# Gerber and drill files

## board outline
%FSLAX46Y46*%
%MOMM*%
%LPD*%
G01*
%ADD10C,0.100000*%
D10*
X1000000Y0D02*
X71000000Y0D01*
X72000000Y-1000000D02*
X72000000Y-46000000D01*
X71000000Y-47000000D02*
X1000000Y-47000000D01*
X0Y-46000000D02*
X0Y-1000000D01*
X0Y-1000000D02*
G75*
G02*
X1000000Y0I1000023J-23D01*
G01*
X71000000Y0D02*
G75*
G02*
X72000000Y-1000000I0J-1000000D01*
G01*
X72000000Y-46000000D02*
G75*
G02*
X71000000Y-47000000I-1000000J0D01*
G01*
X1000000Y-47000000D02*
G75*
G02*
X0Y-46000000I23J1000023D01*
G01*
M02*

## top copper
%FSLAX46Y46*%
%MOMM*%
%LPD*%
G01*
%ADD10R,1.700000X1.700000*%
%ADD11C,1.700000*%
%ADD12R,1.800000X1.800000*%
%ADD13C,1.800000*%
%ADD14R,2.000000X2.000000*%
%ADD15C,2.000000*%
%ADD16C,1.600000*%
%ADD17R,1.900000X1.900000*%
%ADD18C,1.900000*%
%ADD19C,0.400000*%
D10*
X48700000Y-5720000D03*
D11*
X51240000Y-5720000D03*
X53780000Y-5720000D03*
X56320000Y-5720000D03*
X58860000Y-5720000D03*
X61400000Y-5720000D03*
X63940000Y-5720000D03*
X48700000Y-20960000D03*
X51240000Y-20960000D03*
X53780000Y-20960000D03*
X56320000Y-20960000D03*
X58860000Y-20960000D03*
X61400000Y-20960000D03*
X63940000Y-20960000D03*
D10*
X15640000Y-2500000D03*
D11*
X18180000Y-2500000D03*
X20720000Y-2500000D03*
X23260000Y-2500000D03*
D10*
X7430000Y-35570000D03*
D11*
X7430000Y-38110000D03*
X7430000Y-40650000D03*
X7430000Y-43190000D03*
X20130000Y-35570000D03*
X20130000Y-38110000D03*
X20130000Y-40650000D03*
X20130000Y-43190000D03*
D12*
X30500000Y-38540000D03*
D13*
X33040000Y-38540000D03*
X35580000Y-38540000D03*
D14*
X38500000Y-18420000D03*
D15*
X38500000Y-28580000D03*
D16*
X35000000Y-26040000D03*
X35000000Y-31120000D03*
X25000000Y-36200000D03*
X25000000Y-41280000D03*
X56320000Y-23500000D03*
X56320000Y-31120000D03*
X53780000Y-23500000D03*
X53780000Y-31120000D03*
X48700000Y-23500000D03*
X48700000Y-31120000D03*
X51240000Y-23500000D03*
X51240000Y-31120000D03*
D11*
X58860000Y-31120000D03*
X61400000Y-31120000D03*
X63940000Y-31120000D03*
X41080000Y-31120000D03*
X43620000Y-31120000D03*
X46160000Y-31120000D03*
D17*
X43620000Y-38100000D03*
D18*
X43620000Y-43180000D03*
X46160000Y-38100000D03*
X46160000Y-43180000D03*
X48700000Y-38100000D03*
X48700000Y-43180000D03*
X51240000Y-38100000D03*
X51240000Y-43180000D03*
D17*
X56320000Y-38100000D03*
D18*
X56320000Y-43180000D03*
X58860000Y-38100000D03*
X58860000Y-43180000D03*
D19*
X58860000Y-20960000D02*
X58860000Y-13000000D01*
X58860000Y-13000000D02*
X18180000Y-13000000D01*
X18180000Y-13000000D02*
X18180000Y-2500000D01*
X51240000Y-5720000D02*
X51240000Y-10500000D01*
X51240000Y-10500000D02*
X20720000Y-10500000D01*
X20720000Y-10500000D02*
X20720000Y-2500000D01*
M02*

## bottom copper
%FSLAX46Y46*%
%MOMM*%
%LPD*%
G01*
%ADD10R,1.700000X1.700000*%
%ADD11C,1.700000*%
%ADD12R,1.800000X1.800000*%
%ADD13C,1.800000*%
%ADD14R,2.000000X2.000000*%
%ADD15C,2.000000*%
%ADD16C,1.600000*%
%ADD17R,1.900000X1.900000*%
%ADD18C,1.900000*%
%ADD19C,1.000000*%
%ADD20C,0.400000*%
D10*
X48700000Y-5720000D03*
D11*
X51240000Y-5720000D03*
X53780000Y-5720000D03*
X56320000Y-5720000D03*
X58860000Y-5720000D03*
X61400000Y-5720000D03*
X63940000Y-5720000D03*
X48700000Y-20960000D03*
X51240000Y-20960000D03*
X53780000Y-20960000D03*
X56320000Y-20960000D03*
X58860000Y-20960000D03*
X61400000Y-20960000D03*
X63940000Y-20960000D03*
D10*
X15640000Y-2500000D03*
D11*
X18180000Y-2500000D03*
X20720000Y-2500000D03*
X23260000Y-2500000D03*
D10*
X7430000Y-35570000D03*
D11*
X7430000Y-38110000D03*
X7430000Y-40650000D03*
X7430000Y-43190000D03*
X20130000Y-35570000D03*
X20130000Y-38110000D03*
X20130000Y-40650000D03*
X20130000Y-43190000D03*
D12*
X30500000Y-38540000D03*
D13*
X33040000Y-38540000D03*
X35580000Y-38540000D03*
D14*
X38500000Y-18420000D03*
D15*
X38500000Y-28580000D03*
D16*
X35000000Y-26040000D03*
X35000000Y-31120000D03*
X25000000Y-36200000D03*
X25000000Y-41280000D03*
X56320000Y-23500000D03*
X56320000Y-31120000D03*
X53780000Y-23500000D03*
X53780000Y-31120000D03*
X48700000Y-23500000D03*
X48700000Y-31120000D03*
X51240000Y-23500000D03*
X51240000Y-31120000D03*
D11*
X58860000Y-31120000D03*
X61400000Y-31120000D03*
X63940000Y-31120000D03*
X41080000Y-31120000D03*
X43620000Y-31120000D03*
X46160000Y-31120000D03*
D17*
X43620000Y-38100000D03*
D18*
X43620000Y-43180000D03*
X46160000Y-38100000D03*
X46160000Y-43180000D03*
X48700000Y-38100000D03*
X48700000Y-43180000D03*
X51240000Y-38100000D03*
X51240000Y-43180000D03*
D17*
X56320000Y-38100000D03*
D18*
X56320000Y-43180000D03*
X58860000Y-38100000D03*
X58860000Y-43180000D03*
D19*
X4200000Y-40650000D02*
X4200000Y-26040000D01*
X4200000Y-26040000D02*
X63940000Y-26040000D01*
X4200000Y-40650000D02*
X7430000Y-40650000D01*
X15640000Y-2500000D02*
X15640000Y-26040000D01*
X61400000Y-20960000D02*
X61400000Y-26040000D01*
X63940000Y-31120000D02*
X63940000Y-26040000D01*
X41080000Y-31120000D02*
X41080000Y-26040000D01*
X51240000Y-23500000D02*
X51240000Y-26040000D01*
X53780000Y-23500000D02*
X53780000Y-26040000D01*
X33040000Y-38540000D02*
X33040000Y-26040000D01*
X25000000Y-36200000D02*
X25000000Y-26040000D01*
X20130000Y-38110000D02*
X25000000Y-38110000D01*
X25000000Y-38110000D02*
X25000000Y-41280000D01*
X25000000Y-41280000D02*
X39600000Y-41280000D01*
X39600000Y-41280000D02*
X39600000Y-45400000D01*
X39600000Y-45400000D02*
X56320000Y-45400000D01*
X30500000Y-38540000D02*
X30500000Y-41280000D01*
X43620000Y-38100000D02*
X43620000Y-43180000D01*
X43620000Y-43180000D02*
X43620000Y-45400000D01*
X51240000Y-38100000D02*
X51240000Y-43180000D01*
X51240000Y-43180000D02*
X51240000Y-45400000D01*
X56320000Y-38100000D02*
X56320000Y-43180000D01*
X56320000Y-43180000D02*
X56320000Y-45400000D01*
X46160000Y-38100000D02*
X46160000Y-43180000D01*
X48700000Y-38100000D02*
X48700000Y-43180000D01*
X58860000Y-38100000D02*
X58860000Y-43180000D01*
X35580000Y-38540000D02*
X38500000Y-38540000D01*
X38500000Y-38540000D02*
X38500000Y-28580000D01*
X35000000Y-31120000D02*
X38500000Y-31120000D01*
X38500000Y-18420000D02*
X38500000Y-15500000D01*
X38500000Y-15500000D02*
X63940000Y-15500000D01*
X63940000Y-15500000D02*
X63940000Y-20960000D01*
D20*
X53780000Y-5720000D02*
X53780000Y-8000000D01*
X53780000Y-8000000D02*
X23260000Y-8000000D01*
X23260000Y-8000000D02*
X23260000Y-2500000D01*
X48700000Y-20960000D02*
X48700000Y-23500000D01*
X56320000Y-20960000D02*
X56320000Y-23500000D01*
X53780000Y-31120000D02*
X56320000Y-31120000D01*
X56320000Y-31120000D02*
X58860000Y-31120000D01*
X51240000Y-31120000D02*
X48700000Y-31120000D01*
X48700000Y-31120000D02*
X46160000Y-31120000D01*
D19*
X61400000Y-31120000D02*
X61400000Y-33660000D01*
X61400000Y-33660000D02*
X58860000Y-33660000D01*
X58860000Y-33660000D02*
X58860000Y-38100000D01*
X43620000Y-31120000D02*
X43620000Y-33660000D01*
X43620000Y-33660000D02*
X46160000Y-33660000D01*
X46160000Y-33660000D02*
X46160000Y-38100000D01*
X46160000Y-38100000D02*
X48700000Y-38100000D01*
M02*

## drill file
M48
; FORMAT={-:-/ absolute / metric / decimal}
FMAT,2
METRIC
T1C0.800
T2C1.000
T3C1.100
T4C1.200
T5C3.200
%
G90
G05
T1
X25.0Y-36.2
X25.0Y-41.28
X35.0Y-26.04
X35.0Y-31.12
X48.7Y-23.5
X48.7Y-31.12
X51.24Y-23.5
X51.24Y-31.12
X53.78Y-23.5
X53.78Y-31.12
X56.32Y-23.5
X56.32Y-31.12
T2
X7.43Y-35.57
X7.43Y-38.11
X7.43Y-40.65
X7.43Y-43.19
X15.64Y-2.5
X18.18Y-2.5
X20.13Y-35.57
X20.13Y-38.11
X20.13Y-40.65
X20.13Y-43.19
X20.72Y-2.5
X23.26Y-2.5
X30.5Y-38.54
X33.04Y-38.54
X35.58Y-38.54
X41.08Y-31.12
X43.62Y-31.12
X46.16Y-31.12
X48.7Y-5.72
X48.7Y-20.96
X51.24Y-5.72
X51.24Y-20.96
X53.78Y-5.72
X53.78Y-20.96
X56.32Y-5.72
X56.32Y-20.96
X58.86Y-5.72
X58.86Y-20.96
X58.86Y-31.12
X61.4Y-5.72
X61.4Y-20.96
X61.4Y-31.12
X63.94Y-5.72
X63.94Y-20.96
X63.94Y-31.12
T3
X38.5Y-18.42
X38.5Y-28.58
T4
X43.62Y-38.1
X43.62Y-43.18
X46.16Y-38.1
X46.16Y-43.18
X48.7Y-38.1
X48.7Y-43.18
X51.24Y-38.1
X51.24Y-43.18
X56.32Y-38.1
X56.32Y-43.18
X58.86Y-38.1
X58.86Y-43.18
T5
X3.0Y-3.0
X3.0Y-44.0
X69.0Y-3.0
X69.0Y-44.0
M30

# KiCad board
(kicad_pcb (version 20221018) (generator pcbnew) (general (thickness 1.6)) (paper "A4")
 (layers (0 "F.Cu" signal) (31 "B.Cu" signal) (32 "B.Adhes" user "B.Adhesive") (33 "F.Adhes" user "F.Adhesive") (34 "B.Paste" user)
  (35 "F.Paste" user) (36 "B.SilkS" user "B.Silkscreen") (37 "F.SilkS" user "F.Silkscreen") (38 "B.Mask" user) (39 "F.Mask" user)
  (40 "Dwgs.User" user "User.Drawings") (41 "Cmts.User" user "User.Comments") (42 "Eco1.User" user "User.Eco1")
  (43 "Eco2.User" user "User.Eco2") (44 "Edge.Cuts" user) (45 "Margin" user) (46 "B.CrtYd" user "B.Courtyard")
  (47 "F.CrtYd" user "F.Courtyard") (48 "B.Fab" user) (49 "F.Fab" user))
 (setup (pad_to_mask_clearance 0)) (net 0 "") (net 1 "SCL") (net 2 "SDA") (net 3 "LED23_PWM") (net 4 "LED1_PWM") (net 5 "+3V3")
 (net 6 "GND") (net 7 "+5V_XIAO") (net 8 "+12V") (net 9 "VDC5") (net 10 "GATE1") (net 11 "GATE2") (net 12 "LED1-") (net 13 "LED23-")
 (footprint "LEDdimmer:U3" (layer "F.Cu") (at 0 0)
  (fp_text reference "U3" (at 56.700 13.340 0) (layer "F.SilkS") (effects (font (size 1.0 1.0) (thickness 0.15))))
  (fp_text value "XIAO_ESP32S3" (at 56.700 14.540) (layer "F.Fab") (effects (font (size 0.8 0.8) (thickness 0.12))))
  (pad "1" thru_hole rect (at 48.7 5.72) (size 1.7 1.7) (drill 1.0) (layers "*.Cu" "*.Mask"))
  (pad "2" thru_hole circle (at 51.24 5.72) (size 1.7 1.7) (drill 1.0) (layers "*.Cu" "*.Mask") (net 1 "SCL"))
  (pad "3" thru_hole circle (at 53.78 5.72) (size 1.7 1.7) (drill 1.0) (layers "*.Cu" "*.Mask") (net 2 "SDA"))
  (pad "4" thru_hole circle (at 56.32 5.72) (size 1.7 1.7) (drill 1.0) (layers "*.Cu" "*.Mask"))
  (pad "5" thru_hole circle (at 58.86 5.72) (size 1.7 1.7) (drill 1.0) (layers "*.Cu" "*.Mask"))
  (pad "6" thru_hole circle (at 61.4 5.72) (size 1.7 1.7) (drill 1.0) (layers "*.Cu" "*.Mask"))
  (pad "7" thru_hole circle (at 63.94 5.72) (size 1.7 1.7) (drill 1.0) (layers "*.Cu" "*.Mask"))
  (pad "8" thru_hole circle (at 48.7 20.96) (size 1.7 1.7) (drill 1.0) (layers "*.Cu" "*.Mask") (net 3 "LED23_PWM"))
  (pad "9" thru_hole circle (at 51.24 20.96) (size 1.7 1.7) (drill 1.0) (layers "*.Cu" "*.Mask"))
  (pad "10" thru_hole circle (at 53.78 20.96) (size 1.7 1.7) (drill 1.0) (layers "*.Cu" "*.Mask"))
  (pad "11" thru_hole circle (at 56.32 20.96) (size 1.7 1.7) (drill 1.0) (layers "*.Cu" "*.Mask") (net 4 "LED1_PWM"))
  (pad "12" thru_hole circle (at 58.86 20.96) (size 1.7 1.7) (drill 1.0) (layers "*.Cu" "*.Mask") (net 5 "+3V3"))
  (pad "13" thru_hole circle (at 61.4 20.96) (size 1.7 1.7) (drill 1.0) (layers "*.Cu" "*.Mask") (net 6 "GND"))
  (pad "14" thru_hole circle (at 63.94 20.96) (size 1.7 1.7) (drill 1.0) (layers "*.Cu" "*.Mask") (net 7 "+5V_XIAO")))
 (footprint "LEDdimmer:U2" (layer "F.Cu") (at 0 0)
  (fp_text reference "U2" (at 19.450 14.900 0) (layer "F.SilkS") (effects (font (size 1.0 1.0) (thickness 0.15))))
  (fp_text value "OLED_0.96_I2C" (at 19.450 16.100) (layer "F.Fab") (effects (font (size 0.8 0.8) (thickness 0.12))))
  (pad "1" thru_hole rect (at 15.64 2.5) (size 1.7 1.7) (drill 1.0) (layers "*.Cu" "*.Mask") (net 6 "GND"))
  (pad "2" thru_hole circle (at 18.18 2.5) (size 1.7 1.7) (drill 1.0) (layers "*.Cu" "*.Mask") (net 5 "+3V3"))
  (pad "3" thru_hole circle (at 20.72 2.5) (size 1.7 1.7) (drill 1.0) (layers "*.Cu" "*.Mask") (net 1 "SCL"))
  (pad "4" thru_hole circle (at 23.26 2.5) (size 1.7 1.7) (drill 1.0) (layers "*.Cu" "*.Mask") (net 2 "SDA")))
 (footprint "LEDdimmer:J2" (layer "F.Cu") (at 0 0)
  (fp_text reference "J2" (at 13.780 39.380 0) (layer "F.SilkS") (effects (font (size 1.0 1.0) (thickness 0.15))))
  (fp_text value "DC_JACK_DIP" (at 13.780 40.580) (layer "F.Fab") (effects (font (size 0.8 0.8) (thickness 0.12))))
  (pad "1" thru_hole rect (at 7.43 35.57) (size 1.7 1.7) (drill 1.0) (layers "*.Cu" "*.Mask") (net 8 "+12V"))
  (pad "2" thru_hole circle (at 7.43 38.11) (size 1.7 1.7) (drill 1.0) (layers "*.Cu" "*.Mask") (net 8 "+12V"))
  (pad "3" thru_hole circle (at 7.43 40.65) (size 1.7 1.7) (drill 1.0) (layers "*.Cu" "*.Mask") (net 6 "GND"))
  (pad "4" thru_hole circle (at 7.43 43.19) (size 1.7 1.7) (drill 1.0) (layers "*.Cu" "*.Mask") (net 6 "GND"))
  (pad "5" thru_hole circle (at 20.13 35.57) (size 1.7 1.7) (drill 1.0) (layers "*.Cu" "*.Mask") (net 8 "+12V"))
  (pad "6" thru_hole circle (at 20.13 38.11) (size 1.7 1.7) (drill 1.0) (layers "*.Cu" "*.Mask") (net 8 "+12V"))
  (pad "7" thru_hole circle (at 20.13 40.65) (size 1.7 1.7) (drill 1.0) (layers "*.Cu" "*.Mask") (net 6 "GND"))
  (pad "8" thru_hole circle (at 20.13 43.19) (size 1.7 1.7) (drill 1.0) (layers "*.Cu" "*.Mask") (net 6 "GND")))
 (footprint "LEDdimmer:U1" (layer "F.Cu") (at 0 0)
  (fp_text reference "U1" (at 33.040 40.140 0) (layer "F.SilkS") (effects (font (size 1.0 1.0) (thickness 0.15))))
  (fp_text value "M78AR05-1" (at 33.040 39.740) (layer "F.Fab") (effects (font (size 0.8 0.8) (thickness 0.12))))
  (pad "1" thru_hole rect (at 30.5 38.54) (size 1.8 1.8) (drill 1.0) (layers "*.Cu" "*.Mask") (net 8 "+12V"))
  (pad "2" thru_hole circle (at 33.04 38.54) (size 1.8 1.8) (drill 1.0) (layers "*.Cu" "*.Mask") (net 6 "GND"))
  (pad "3" thru_hole circle (at 35.58 38.54) (size 1.8 1.8) (drill 1.0) (layers "*.Cu" "*.Mask") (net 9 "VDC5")))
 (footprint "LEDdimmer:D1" (layer "F.Cu") (at 0 0)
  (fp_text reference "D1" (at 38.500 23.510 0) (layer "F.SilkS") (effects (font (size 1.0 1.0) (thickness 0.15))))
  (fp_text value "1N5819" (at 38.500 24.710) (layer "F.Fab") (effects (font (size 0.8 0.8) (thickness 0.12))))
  (pad "1" thru_hole rect (at 38.5 18.42) (size 2.0 2.0) (drill 1.1) (layers "*.Cu" "*.Mask") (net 7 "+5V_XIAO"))
  (pad "2" thru_hole circle (at 38.5 28.58) (size 2.0 2.0) (drill 1.1) (layers "*.Cu" "*.Mask") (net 9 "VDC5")))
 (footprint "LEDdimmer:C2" (layer "F.Cu") (at 0 0)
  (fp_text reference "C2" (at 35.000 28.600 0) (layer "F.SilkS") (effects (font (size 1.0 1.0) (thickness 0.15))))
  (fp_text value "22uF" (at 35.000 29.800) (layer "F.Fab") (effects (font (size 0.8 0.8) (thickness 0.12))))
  (pad "1" thru_hole circle (at 35.0 26.04) (size 1.6 1.6) (drill 0.8) (layers "*.Cu" "*.Mask") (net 6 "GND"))
  (pad "2" thru_hole circle (at 35.0 31.12) (size 1.6 1.6) (drill 0.8) (layers "*.Cu" "*.Mask") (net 9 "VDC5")))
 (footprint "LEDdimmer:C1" (layer "F.Cu") (at 0 0)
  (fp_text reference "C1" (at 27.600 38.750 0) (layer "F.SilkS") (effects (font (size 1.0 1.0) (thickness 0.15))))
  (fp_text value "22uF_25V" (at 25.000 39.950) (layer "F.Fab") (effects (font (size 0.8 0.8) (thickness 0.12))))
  (pad "1" thru_hole circle (at 25.0 36.2) (size 1.6 1.6) (drill 0.8) (layers "*.Cu" "*.Mask") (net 6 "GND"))
  (pad "2" thru_hole circle (at 25.0 41.28) (size 1.6 1.6) (drill 0.8) (layers "*.Cu" "*.Mask") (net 8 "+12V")))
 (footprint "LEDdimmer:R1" (layer "F.Cu") (at 0 0)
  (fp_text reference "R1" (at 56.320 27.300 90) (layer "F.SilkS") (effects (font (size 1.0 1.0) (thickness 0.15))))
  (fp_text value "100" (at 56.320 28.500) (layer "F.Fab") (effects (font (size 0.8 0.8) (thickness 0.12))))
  (pad "1" thru_hole circle (at 56.32 23.5) (size 1.6 1.6) (drill 0.8) (layers "*.Cu" "*.Mask") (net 4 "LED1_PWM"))
  (pad "2" thru_hole circle (at 56.32 31.12) (size 1.6 1.6) (drill 0.8) (layers "*.Cu" "*.Mask") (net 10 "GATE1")))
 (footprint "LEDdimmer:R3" (layer "F.Cu") (at 0 0)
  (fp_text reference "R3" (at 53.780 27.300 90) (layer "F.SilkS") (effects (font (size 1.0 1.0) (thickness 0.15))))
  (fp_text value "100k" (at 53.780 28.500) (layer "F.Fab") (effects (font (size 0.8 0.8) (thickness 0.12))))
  (pad "1" thru_hole circle (at 53.78 23.5) (size 1.6 1.6) (drill 0.8) (layers "*.Cu" "*.Mask") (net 6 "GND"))
  (pad "2" thru_hole circle (at 53.78 31.12) (size 1.6 1.6) (drill 0.8) (layers "*.Cu" "*.Mask") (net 10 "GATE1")))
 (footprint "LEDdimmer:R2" (layer "F.Cu") (at 0 0)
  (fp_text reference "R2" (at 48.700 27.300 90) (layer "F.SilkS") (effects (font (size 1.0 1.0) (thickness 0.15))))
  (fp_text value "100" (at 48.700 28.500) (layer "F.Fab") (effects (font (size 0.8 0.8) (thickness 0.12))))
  (pad "1" thru_hole circle (at 48.7 23.5) (size 1.6 1.6) (drill 0.8) (layers "*.Cu" "*.Mask") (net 3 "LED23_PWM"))
  (pad "2" thru_hole circle (at 48.7 31.12) (size 1.6 1.6) (drill 0.8) (layers "*.Cu" "*.Mask") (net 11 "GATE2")))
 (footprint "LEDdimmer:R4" (layer "F.Cu") (at 0 0)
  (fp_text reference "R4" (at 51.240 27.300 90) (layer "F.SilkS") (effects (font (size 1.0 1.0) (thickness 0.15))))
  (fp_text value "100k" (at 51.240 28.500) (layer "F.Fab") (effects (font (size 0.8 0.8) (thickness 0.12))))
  (pad "1" thru_hole circle (at 51.24 23.5) (size 1.6 1.6) (drill 0.8) (layers "*.Cu" "*.Mask") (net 6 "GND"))
  (pad "2" thru_hole circle (at 51.24 31.12) (size 1.6 1.6) (drill 0.8) (layers "*.Cu" "*.Mask") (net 11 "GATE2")))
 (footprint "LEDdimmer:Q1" (layer "F.Cu") (at 0 0)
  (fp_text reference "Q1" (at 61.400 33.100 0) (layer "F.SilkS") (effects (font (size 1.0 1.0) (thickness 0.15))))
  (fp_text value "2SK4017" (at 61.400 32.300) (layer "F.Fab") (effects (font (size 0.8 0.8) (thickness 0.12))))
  (pad "1" thru_hole circle (at 58.86 31.12) (size 1.7 1.7) (drill 1.0) (layers "*.Cu" "*.Mask") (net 10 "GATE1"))
  (pad "2" thru_hole circle (at 61.4 31.12) (size 1.7 1.7) (drill 1.0) (layers "*.Cu" "*.Mask") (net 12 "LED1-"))
  (pad "3" thru_hole circle (at 63.94 31.12) (size 1.7 1.7) (drill 1.0) (layers "*.Cu" "*.Mask") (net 6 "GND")))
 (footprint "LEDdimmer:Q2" (layer "F.Cu") (at 0 0)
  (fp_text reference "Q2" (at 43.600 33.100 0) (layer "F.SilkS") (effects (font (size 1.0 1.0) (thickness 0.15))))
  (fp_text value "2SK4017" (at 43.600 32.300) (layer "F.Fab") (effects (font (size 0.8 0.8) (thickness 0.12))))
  (pad "1" thru_hole circle (at 41.08 31.12) (size 1.7 1.7) (drill 1.0) (layers "*.Cu" "*.Mask") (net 6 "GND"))
  (pad "2" thru_hole circle (at 43.62 31.12) (size 1.7 1.7) (drill 1.0) (layers "*.Cu" "*.Mask") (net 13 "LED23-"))
  (pad "3" thru_hole circle (at 46.16 31.12) (size 1.7 1.7) (drill 1.0) (layers "*.Cu" "*.Mask") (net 11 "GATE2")))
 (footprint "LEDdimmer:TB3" (layer "F.Cu") (at 0 0)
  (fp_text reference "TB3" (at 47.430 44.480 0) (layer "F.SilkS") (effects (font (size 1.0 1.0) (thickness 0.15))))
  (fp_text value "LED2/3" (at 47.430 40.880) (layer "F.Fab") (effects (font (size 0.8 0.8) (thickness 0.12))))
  (pad "1" thru_hole rect (at 43.62 38.1) (size 1.9 1.9) (drill 1.2) (layers "*.Cu" "*.Mask") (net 8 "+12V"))
  (pad "2" thru_hole circle (at 43.62 43.18) (size 1.9 1.9) (drill 1.2) (layers "*.Cu" "*.Mask") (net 8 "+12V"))
  (pad "3" thru_hole circle (at 46.16 38.1) (size 1.9 1.9) (drill 1.2) (layers "*.Cu" "*.Mask") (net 13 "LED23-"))
  (pad "4" thru_hole circle (at 46.16 43.18) (size 1.9 1.9) (drill 1.2) (layers "*.Cu" "*.Mask") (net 13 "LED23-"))
  (pad "5" thru_hole circle (at 48.7 38.1) (size 1.9 1.9) (drill 1.2) (layers "*.Cu" "*.Mask") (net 13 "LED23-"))
  (pad "6" thru_hole circle (at 48.7 43.18) (size 1.9 1.9) (drill 1.2) (layers "*.Cu" "*.Mask") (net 13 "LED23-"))
  (pad "7" thru_hole circle (at 51.24 38.1) (size 1.9 1.9) (drill 1.2) (layers "*.Cu" "*.Mask") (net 8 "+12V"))
  (pad "8" thru_hole circle (at 51.24 43.18) (size 1.9 1.9) (drill 1.2) (layers "*.Cu" "*.Mask") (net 8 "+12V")))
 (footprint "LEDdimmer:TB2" (layer "F.Cu") (at 0 0)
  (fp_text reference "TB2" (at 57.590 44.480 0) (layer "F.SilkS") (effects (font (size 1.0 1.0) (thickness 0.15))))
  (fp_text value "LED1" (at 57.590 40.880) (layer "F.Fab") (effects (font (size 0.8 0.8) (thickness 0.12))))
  (pad "1" thru_hole rect (at 56.32 38.1) (size 1.9 1.9) (drill 1.2) (layers "*.Cu" "*.Mask") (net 8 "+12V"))
  (pad "2" thru_hole circle (at 56.32 43.18) (size 1.9 1.9) (drill 1.2) (layers "*.Cu" "*.Mask") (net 8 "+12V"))
  (pad "3" thru_hole circle (at 58.86 38.1) (size 1.9 1.9) (drill 1.2) (layers "*.Cu" "*.Mask") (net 12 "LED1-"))
  (pad "4" thru_hole circle (at 58.86 43.18) (size 1.9 1.9) (drill 1.2) (layers "*.Cu" "*.Mask") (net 12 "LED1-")))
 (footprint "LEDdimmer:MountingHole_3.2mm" (layer "F.Cu") (at 3.0 3.0)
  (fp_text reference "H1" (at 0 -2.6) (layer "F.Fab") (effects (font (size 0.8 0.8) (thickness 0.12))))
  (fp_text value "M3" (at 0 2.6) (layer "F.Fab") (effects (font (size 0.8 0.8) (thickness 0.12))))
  (pad "" np_thru_hole circle (at 0 0) (size 3.2 3.2) (drill 3.2) (layers "*.Cu" "*.Mask")))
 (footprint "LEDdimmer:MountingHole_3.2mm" (layer "F.Cu") (at 69.0 3.0)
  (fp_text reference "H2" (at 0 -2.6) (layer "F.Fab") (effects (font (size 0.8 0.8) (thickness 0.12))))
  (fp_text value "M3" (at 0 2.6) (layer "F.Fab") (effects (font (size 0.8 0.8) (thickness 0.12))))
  (pad "" np_thru_hole circle (at 0 0) (size 3.2 3.2) (drill 3.2) (layers "*.Cu" "*.Mask")))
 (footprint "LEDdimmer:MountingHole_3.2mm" (layer "F.Cu") (at 3.0 44.0)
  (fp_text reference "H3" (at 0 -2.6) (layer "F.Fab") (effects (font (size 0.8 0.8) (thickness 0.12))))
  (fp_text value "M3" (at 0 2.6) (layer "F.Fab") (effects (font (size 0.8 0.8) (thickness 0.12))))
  (pad "" np_thru_hole circle (at 0 0) (size 3.2 3.2) (drill 3.2) (layers "*.Cu" "*.Mask")))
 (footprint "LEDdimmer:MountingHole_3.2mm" (layer "F.Cu") (at 69.0 44.0)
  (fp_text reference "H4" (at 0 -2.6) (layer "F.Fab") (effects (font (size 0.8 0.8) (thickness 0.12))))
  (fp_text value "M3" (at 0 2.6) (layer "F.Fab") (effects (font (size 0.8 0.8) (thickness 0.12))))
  (pad "" np_thru_hole circle (at 0 0) (size 3.2 3.2) (drill 3.2) (layers "*.Cu" "*.Mask")))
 (gr_line (start 1.0 0) (end 71.0 0) (stroke (width 0.1) (type solid)) (layer "Edge.Cuts"))
 (gr_line (start 72.0 1.0) (end 72.0 46.0) (stroke (width 0.1) (type solid)) (layer "Edge.Cuts"))
 (gr_line (start 71.0 47.0) (end 1.0 47.0) (stroke (width 0.1) (type solid)) (layer "Edge.Cuts"))
 (gr_line (start 0 46.0) (end 0 1.0) (stroke (width 0.1) (type solid)) (layer "Edge.Cuts"))
 (gr_arc (start 1.0 0) (mid 0.2929 0.2929) (end 0 1.0) (stroke (width 0.1) (type solid)) (layer "Edge.Cuts"))
 (gr_arc (start 72.0 1.0) (mid 71.7071 0.2929) (end 71.0 0) (stroke (width 0.1) (type solid)) (layer "Edge.Cuts"))
 (gr_arc (start 71.0 47.0) (mid 71.7071 46.7071) (end 72.0 46.0) (stroke (width 0.1) (type solid)) (layer "Edge.Cuts"))
 (gr_arc (start 0 46.0) (mid 0.2929 46.7071) (end 1.0 47.0) (stroke (width 0.1) (type solid)) (layer "Edge.Cuts"))
 (segment (start 4.2 40.65) (end 4.2 26.04) (width 1.0) (layer "B.Cu") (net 6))
 (segment (start 4.2 26.04) (end 63.94 26.04) (width 1.0) (layer "B.Cu") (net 6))
 (segment (start 4.2 40.65) (end 7.43 40.65) (width 1.0) (layer "B.Cu") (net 6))
 (segment (start 15.64 2.5) (end 15.64 26.04) (width 1.0) (layer "B.Cu") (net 6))
 (segment (start 61.4 20.96) (end 61.4 26.04) (width 1.0) (layer "B.Cu") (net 6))
 (segment (start 63.94 31.12) (end 63.94 26.04) (width 1.0) (layer "B.Cu") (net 6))
 (segment (start 41.08 31.12) (end 41.08 26.04) (width 1.0) (layer "B.Cu") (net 6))
 (segment (start 51.24 23.5) (end 51.24 26.04) (width 1.0) (layer "B.Cu") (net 6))
 (segment (start 53.78 23.5) (end 53.78 26.04) (width 1.0) (layer "B.Cu") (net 6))
 (segment (start 33.04 38.54) (end 33.04 26.04) (width 1.0) (layer "B.Cu") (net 6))
 (segment (start 25.0 36.2) (end 25.0 26.04) (width 1.0) (layer "B.Cu") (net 6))
 (segment (start 20.13 38.11) (end 25.0 38.11) (width 1.0) (layer "B.Cu") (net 8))
 (segment (start 25.0 38.11) (end 25.0 41.28) (width 1.0) (layer "B.Cu") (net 8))
 (segment (start 25.0 41.28) (end 39.6 41.28) (width 1.0) (layer "B.Cu") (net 8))
 (segment (start 39.6 41.28) (end 39.6 45.4) (width 1.0) (layer "B.Cu") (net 8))
 (segment (start 39.6 45.4) (end 56.32 45.4) (width 1.0) (layer "B.Cu") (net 8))
 (segment (start 30.5 38.54) (end 30.5 41.28) (width 1.0) (layer "B.Cu") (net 8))
 (segment (start 43.62 38.1) (end 43.62 43.18) (width 1.0) (layer "B.Cu") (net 8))
 (segment (start 43.62 43.18) (end 43.62 45.4) (width 1.0) (layer "B.Cu") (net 8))
 (segment (start 51.24 38.1) (end 51.24 43.18) (width 1.0) (layer "B.Cu") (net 8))
 (segment (start 51.24 43.18) (end 51.24 45.4) (width 1.0) (layer "B.Cu") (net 8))
 (segment (start 56.32 38.1) (end 56.32 43.18) (width 1.0) (layer "B.Cu") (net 8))
 (segment (start 56.32 43.18) (end 56.32 45.4) (width 1.0) (layer "B.Cu") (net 8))
 (segment (start 46.16 38.1) (end 46.16 43.18) (width 1.0) (layer "B.Cu") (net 13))
 (segment (start 48.7 38.1) (end 48.7 43.18) (width 1.0) (layer "B.Cu") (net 13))
 (segment (start 58.86 38.1) (end 58.86 43.18) (width 1.0) (layer "B.Cu") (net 12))
 (segment (start 35.58 38.54) (end 38.5 38.54) (width 1.0) (layer "B.Cu") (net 9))
 (segment (start 38.5 38.54) (end 38.5 28.58) (width 1.0) (layer "B.Cu") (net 9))
 (segment (start 35.0 31.12) (end 38.5 31.12) (width 1.0) (layer "B.Cu") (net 9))
 (segment (start 38.5 18.42) (end 38.5 15.5) (width 1.0) (layer "B.Cu") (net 7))
 (segment (start 38.5 15.5) (end 63.94 15.5) (width 1.0) (layer "B.Cu") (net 7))
 (segment (start 63.94 15.5) (end 63.94 20.96) (width 1.0) (layer "B.Cu") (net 7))
 (segment (start 58.86 20.96) (end 58.86 13.0) (width 0.4) (layer "F.Cu") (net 5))
 (segment (start 58.86 13.0) (end 18.18 13.0) (width 0.4) (layer "F.Cu") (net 5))
 (segment (start 18.18 13.0) (end 18.18 2.5) (width 0.4) (layer "F.Cu") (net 5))
 (segment (start 51.24 5.72) (end 51.24 10.5) (width 0.4) (layer "F.Cu") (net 1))
 (segment (start 51.24 10.5) (end 20.72 10.5) (width 0.4) (layer "F.Cu") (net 1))
 (segment (start 20.72 10.5) (end 20.72 2.5) (width 0.4) (layer "F.Cu") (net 1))
 (segment (start 53.78 5.72) (end 53.78 8.0) (width 0.4) (layer "B.Cu") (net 2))
 (segment (start 53.78 8.0) (end 23.26 8.0) (width 0.4) (layer "B.Cu") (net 2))
 (segment (start 23.26 8.0) (end 23.26 2.5) (width 0.4) (layer "B.Cu") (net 2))
 (segment (start 48.7 20.96) (end 48.7 23.5) (width 0.4) (layer "B.Cu") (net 3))
 (segment (start 56.32 20.96) (end 56.32 23.5) (width 0.4) (layer "B.Cu") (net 4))
 (segment (start 53.78 31.12) (end 56.32 31.12) (width 0.4) (layer "B.Cu") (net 10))
 (segment (start 56.32 31.12) (end 58.86 31.12) (width 0.4) (layer "B.Cu") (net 10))
 (segment (start 51.24 31.12) (end 48.7 31.12) (width 0.4) (layer "B.Cu") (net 11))
 (segment (start 48.7 31.12) (end 46.16 31.12) (width 0.4) (layer "B.Cu") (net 11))
 (segment (start 61.4 31.12) (end 61.4 33.66) (width 1.0) (layer "B.Cu") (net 12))
 (segment (start 61.4 33.66) (end 58.86 33.66) (width 1.0) (layer "B.Cu") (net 12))
 (segment (start 58.86 33.66) (end 58.86 38.1) (width 1.0) (layer "B.Cu") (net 12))
 (segment (start 43.62 31.12) (end 43.62 33.66) (width 1.0) (layer "B.Cu") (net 13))
 (segment (start 43.62 33.66) (end 46.16 33.66) (width 1.0) (layer "B.Cu") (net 13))
 (segment (start 46.16 33.66) (end 46.16 38.1) (width 1.0) (layer "B.Cu") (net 13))
 (segment (start 46.16 38.1) (end 48.7 38.1) (width 1.0) (layer "B.Cu") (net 13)))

